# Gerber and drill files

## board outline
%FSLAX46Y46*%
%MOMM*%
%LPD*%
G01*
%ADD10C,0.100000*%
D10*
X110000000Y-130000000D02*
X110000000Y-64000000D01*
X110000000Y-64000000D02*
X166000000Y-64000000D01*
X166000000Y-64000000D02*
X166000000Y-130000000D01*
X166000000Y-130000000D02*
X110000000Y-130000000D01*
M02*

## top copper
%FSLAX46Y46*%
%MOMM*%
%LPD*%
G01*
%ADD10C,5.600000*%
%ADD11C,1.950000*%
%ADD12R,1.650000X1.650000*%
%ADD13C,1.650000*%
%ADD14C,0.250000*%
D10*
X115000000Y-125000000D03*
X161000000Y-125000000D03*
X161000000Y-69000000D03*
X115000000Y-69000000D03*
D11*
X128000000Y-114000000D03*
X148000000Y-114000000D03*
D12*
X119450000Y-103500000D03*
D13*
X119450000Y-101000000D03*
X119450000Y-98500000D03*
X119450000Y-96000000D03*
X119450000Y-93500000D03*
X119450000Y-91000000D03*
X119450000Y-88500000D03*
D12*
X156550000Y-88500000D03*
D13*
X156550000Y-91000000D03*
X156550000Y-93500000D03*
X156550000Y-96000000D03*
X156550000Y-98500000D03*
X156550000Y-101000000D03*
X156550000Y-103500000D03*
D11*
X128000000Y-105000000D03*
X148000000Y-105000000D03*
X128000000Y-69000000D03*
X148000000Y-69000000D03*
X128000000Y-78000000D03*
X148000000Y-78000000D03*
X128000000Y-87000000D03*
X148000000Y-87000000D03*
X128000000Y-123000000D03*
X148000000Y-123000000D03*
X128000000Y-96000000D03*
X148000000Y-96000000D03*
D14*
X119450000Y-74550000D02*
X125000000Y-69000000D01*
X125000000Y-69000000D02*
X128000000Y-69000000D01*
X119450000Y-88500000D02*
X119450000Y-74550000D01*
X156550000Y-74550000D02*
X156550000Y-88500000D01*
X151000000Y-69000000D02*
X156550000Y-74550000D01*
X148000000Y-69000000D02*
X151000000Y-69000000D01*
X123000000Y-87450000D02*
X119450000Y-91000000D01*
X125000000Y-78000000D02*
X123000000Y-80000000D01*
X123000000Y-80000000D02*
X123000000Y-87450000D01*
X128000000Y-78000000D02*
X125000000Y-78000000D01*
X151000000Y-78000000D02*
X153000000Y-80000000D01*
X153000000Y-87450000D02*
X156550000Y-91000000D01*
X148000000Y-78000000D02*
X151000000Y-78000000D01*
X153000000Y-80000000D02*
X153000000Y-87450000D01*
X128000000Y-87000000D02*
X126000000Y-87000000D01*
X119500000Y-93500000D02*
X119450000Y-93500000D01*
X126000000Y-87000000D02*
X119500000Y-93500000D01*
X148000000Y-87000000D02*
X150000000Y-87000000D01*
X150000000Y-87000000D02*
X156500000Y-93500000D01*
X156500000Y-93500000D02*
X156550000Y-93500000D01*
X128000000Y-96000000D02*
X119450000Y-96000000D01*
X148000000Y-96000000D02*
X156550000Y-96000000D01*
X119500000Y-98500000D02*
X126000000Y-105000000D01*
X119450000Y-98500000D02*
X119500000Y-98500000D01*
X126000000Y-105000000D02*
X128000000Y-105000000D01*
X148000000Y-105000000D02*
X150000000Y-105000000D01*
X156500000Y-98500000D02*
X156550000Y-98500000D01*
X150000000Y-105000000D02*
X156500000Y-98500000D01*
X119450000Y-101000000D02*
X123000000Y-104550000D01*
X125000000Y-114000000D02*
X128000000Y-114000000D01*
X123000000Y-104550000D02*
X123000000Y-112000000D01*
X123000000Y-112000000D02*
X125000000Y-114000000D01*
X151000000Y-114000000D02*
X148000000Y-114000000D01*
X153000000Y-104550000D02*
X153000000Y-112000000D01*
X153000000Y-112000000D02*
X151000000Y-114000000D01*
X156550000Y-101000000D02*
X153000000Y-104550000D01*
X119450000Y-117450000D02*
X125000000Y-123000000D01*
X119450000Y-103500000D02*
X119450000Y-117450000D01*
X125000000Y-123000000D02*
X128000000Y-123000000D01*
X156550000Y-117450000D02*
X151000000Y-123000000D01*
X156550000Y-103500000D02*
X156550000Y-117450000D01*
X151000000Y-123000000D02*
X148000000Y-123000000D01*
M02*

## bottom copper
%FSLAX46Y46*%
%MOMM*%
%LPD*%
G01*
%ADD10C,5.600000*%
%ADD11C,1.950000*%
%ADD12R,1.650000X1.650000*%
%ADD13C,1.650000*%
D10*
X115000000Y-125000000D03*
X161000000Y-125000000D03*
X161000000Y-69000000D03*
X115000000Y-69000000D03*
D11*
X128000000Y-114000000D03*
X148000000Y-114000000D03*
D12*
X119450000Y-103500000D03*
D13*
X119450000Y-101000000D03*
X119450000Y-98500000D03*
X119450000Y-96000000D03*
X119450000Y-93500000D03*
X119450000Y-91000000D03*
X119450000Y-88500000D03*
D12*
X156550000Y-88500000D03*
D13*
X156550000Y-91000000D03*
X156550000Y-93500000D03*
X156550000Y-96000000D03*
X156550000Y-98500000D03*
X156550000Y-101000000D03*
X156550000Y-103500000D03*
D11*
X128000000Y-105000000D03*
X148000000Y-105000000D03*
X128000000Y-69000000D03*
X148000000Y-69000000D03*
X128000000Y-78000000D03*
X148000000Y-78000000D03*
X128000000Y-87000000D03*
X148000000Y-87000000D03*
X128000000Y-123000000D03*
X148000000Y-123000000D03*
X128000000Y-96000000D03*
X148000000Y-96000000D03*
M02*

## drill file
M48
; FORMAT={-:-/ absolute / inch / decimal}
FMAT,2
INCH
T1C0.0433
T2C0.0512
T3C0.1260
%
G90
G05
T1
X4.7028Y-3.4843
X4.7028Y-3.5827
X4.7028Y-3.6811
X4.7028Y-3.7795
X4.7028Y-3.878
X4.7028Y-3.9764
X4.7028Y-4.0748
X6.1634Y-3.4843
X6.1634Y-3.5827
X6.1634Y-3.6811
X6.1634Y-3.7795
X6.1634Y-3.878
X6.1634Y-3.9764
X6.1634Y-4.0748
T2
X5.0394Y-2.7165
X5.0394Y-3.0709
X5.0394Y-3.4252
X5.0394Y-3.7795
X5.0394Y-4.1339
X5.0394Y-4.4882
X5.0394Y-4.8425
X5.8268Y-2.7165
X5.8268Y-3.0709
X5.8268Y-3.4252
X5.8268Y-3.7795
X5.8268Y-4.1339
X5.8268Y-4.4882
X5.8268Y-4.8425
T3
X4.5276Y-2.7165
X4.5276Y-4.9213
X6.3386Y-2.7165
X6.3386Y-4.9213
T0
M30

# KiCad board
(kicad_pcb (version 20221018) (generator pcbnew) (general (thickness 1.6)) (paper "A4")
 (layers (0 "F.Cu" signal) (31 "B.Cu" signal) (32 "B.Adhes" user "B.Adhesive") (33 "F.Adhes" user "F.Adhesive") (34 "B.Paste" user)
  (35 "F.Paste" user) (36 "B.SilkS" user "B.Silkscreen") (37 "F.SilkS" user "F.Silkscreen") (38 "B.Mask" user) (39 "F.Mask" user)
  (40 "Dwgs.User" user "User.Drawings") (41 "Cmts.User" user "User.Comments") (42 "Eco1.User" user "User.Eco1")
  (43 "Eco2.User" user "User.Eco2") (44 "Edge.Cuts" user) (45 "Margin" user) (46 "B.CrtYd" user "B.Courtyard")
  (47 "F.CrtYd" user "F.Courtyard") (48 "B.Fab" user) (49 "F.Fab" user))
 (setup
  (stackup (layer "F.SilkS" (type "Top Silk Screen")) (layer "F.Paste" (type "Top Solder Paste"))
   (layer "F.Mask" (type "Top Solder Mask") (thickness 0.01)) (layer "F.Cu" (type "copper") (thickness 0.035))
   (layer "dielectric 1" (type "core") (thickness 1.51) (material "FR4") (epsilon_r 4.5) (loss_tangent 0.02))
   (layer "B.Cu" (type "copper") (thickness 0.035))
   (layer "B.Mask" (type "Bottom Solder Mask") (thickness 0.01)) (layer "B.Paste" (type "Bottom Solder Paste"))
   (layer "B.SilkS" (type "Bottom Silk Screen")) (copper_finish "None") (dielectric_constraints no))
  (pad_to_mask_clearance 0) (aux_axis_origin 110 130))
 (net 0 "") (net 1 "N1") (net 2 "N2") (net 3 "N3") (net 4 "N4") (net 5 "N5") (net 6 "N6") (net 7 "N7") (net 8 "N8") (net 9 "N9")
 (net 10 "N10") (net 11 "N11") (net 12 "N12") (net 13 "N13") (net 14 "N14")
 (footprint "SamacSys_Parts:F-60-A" (layer "F.Cu") (at 138 114)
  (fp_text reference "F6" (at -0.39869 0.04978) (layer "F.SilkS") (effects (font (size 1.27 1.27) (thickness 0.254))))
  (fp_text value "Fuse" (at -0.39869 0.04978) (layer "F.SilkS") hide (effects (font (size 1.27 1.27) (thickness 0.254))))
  (pad "1" thru_hole circle (at -10 0) (size 1.95 1.95) (drill 1.3) (layers "*.Cu" "*.Mask") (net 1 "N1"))
  (pad "2" thru_hole circle (at 10 0) (size 1.95 1.95) (drill 1.3) (layers "*.Cu" "*.Mask") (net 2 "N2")))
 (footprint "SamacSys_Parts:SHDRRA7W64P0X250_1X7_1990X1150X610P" (layer "F.Cu") (at 119.45 103.5 90)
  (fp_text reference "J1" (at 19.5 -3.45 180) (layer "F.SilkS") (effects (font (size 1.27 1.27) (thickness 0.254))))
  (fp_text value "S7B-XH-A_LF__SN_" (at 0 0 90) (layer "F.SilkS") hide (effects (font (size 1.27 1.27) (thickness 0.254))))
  (pad "1" thru_hole rect (at 0 0 90) (size 1.65 1.65) (drill 1.1) (layers "*.Cu" "*.Mask") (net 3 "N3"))
  (pad "2" thru_hole circle (at 2.5 0 90) (size 1.65 1.65) (drill 1.1) (layers "*.Cu" "*.Mask") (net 1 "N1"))
  (pad "3" thru_hole circle (at 5 0 90) (size 1.65 1.65) (drill 1.1) (layers "*.Cu" "*.Mask") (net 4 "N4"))
  (pad "4" thru_hole circle (at 7.5 0 90) (size 1.65 1.65) (drill 1.1) (layers "*.Cu" "*.Mask") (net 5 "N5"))
  (pad "5" thru_hole circle (at 10 0 90) (size 1.65 1.65) (drill 1.1) (layers "*.Cu" "*.Mask") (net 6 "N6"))
  (pad "6" thru_hole circle (at 12.5 0 90) (size 1.65 1.65) (drill 1.1) (layers "*.Cu" "*.Mask") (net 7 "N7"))
  (pad "7" thru_hole circle (at 15 0 90) (size 1.65 1.65) (drill 1.1) (layers "*.Cu" "*.Mask") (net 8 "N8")))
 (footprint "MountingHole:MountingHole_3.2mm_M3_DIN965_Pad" (layer "F.Cu") (at 161 69)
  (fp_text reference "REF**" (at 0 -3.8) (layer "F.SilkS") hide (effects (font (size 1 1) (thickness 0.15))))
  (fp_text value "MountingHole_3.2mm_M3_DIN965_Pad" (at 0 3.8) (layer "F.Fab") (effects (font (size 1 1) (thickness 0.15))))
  (pad "1" thru_hole circle (at 0 0) (size 5.6 5.6) (drill 3.2) (layers "F&B.Cu" "*.Mask")))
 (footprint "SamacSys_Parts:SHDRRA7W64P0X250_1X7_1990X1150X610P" (layer "F.Cu") (at 156.55 88.5 -90)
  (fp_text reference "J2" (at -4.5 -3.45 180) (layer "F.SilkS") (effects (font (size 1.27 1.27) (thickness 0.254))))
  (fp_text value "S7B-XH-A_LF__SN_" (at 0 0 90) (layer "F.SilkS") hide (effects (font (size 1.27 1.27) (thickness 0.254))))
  (pad "1" thru_hole rect (at 0 0 270) (size 1.65 1.65) (drill 1.1) (layers "*.Cu" "*.Mask") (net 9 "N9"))
  (pad "2" thru_hole circle (at 2.5 0 270) (size 1.65 1.65) (drill 1.1) (layers "*.Cu" "*.Mask") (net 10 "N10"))
  (pad "3" thru_hole circle (at 5 0 270) (size 1.65 1.65) (drill 1.1) (layers "*.Cu" "*.Mask") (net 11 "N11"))
  (pad "4" thru_hole circle (at 7.5 0 270) (size 1.65 1.65) (drill 1.1) (layers "*.Cu" "*.Mask") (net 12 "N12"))
  (pad "5" thru_hole circle (at 10 0 270) (size 1.65 1.65) (drill 1.1) (layers "*.Cu" "*.Mask") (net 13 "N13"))
  (pad "6" thru_hole circle (at 12.5 0 270) (size 1.65 1.65) (drill 1.1) (layers "*.Cu" "*.Mask") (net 2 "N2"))
  (pad "7" thru_hole circle (at 15 0 270) (size 1.65 1.65) (drill 1.1) (layers "*.Cu" "*.Mask") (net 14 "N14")))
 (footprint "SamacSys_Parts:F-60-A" (layer "F.Cu") (at 138 105)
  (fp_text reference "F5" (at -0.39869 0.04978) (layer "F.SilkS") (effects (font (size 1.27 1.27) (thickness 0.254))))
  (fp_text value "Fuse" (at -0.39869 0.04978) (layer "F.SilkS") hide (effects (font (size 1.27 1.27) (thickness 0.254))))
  (pad "1" thru_hole circle (at -10 0) (size 1.95 1.95) (drill 1.3) (layers "*.Cu" "*.Mask") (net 4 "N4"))
  (pad "2" thru_hole circle (at 10 0) (size 1.95 1.95) (drill 1.3) (layers "*.Cu" "*.Mask") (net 13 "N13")))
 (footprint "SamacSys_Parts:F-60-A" (layer "F.Cu") (at 138 69)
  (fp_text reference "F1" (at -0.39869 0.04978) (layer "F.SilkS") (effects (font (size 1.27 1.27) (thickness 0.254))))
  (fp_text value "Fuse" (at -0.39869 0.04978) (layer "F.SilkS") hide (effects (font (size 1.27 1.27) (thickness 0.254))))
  (pad "1" thru_hole circle (at -10 0) (size 1.95 1.95) (drill 1.3) (layers "*.Cu" "*.Mask") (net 8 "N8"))
  (pad "2" thru_hole circle (at 10 0) (size 1.95 1.95) (drill 1.3) (layers "*.Cu" "*.Mask") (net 9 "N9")))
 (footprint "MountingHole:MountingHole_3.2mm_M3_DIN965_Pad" (layer "F.Cu") (at 115 125)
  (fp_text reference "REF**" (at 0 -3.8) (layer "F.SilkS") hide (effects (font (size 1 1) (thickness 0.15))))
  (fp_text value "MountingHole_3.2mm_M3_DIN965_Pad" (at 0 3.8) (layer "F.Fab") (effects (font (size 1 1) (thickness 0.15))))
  (pad "1" thru_hole circle (at 0 0) (size 5.6 5.6) (drill 3.2) (layers "F&B.Cu" "*.Mask")))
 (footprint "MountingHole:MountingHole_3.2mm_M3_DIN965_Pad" (layer "F.Cu") (at 115 69)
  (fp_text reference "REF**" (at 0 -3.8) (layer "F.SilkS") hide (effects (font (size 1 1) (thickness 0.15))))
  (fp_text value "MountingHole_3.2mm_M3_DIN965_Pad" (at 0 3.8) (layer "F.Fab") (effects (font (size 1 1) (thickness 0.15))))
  (pad "1" thru_hole circle (at 0 0) (size 5.6 5.6) (drill 3.2) (layers "*.Cu" "*.Mask")))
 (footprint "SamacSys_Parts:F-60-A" (layer "F.Cu") (at 138 78)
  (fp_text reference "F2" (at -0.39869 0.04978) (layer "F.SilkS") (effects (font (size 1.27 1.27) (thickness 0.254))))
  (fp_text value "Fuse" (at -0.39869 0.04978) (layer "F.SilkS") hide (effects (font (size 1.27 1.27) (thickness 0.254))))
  (pad "1" thru_hole circle (at -10 0) (size 1.95 1.95) (drill 1.3) (layers "*.Cu" "*.Mask") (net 7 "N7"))
  (pad "2" thru_hole circle (at 10 0) (size 1.95 1.95) (drill 1.3) (layers "*.Cu" "*.Mask") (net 10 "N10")))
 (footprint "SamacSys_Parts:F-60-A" (layer "F.Cu") (at 138 87)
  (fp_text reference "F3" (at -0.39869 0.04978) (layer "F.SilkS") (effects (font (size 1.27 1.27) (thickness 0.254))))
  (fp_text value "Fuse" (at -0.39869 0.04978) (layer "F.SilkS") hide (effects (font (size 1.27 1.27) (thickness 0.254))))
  (pad "1" thru_hole circle (at -10 0) (size 1.95 1.95) (drill 1.3) (layers "*.Cu" "*.Mask") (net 6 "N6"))
  (pad "2" thru_hole circle (at 10 0) (size 1.95 1.95) (drill 1.3) (layers "*.Cu" "*.Mask") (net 11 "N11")))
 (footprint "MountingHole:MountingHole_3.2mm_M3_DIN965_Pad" (layer "F.Cu") (at 161 125)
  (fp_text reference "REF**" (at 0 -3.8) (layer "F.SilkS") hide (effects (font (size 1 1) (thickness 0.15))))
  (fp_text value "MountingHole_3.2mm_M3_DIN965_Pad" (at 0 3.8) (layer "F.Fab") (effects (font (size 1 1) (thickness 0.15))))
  (pad "1" thru_hole circle (at 0 0) (size 5.6 5.6) (drill 3.2) (layers "F&B.Cu" "*.Mask")))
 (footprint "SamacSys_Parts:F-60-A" (layer "F.Cu") (at 138 123)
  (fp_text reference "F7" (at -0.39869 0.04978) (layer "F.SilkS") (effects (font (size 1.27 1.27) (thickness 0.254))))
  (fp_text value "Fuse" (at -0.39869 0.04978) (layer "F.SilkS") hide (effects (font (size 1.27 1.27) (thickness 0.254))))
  (pad "1" thru_hole circle (at -10 0) (size 1.95 1.95) (drill 1.3) (layers "*.Cu" "*.Mask") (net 3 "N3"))
  (pad "2" thru_hole circle (at 10 0) (size 1.95 1.95) (drill 1.3) (layers "*.Cu" "*.Mask") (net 14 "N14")))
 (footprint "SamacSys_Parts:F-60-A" (layer "F.Cu") (at 138 96)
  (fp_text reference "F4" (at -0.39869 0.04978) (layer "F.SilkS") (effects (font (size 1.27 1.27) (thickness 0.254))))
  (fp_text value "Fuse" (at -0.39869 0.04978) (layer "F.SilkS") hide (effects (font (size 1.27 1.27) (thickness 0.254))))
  (pad "1" thru_hole circle (at -10 0) (size 1.95 1.95) (drill 1.3) (layers "*.Cu" "*.Mask") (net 5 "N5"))
  (pad "2" thru_hole circle (at 10 0) (size 1.95 1.95) (drill 1.3) (layers "*.Cu" "*.Mask") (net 12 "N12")))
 (gr_line (start 110 130) (end 110 64) (stroke (width 0.1) (type solid)) (layer "Edge.Cuts"))
 (gr_line (start 110 64) (end 166 64) (stroke (width 0.1) (type solid)) (layer "Edge.Cuts"))
 (gr_line (start 166 64) (end 166 130) (stroke (width 0.1) (type solid)) (layer "Edge.Cuts"))
 (gr_line (start 166 130) (end 110 130) (stroke (width 0.1) (type solid)) (layer "Edge.Cuts"))
 (segment (start 119.45 74.55) (end 125 69) (width 0.25) (layer "F.Cu") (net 8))
 (segment (start 125 69) (end 128 69) (width 0.25) (layer "F.Cu") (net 8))
 (segment (start 119.45 88.5) (end 119.45 74.55) (width 0.25) (layer "F.Cu") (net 8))
 (segment (start 156.55 74.55) (end 156.55 88.5) (width 0.25) (layer "F.Cu") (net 9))
 (segment (start 151 69) (end 156.55 74.55) (width 0.25) (layer "F.Cu") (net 9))
 (segment (start 148 69) (end 151 69) (width 0.25) (layer "F.Cu") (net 9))
 (segment (start 123 87.45) (end 119.45 91) (width 0.25) (layer "F.Cu") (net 7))
 (segment (start 125 78) (end 123 80) (width 0.25) (layer "F.Cu") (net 7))
 (segment (start 123 80) (end 123 87.45) (width 0.25) (layer "F.Cu") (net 7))
 (segment (start 128 78) (end 125 78) (width 0.25) (layer "F.Cu") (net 7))
 (segment (start 151 78) (end 153 80) (width 0.25) (layer "F.Cu") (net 10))
 (segment (start 153 87.45) (end 156.55 91) (width 0.25) (layer "F.Cu") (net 10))
 (segment (start 148 78) (end 151 78) (width 0.25) (layer "F.Cu") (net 10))
 (segment (start 153 80) (end 153 87.45) (width 0.25) (layer "F.Cu") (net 10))
 (segment (start 128 87) (end 126 87) (width 0.25) (layer "F.Cu") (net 6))
 (segment (start 119.5 93.5) (end 119.45 93.5) (width 0.25) (layer "F.Cu") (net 6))
 (segment (start 126 87) (end 119.5 93.5) (width 0.25) (layer "F.Cu") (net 6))
 (segment (start 148 87) (end 150 87) (width 0.25) (layer "F.Cu") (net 11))
 (segment (start 150 87) (end 156.5 93.5) (width 0.25) (layer "F.Cu") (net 11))
 (segment (start 156.5 93.5) (end 156.55 93.5) (width 0.25) (layer "F.Cu") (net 11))
 (segment (start 128 96) (end 119.45 96) (width 0.25) (layer "F.Cu") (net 5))
 (segment (start 148 96) (end 156.55 96) (width 0.25) (layer "F.Cu") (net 12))
 (segment (start 119.5 98.5) (end 126 105) (width 0.25) (layer "F.Cu") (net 4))
 (segment (start 119.45 98.5) (end 119.5 98.5) (width 0.25) (layer "F.Cu") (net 4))
 (segment (start 126 105) (end 128 105) (width 0.25) (layer "F.Cu") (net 4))
 (segment (start 148 105) (end 150 105) (width 0.25) (layer "F.Cu") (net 13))
 (segment (start 156.5 98.5) (end 156.55 98.5) (width 0.25) (layer "F.Cu") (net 13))
 (segment (start 150 105) (end 156.5 98.5) (width 0.25) (layer "F.Cu") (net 13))
 (segment (start 119.45 101) (end 123 104.55) (width 0.25) (layer "F.Cu") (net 1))
 (segment (start 125 114) (end 128 114) (width 0.25) (layer "F.Cu") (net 1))
 (segment (start 123 104.55) (end 123 112) (width 0.25) (layer "F.Cu") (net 1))
 (segment (start 123 112) (end 125 114) (width 0.25) (layer "F.Cu") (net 1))
 (segment (start 151 114) (end 148 114) (width 0.25) (layer "F.Cu") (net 2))
 (segment (start 153 104.55) (end 153 112) (width 0.25) (layer "F.Cu") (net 2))
 (segment (start 153 112) (end 151 114) (width 0.25) (layer "F.Cu") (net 2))
 (segment (start 156.55 101) (end 153 104.55) (width 0.25) (layer "F.Cu") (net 2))
 (segment (start 119.45 117.45) (end 125 123) (width 0.25) (layer "F.Cu") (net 3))
 (segment (start 119.45 103.5) (end 119.45 117.45) (width 0.25) (layer "F.Cu") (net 3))
 (segment (start 125 123) (end 128 123) (width 0.25) (layer "F.Cu") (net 3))
 (segment (start 156.55 117.45) (end 151 123) (width 0.25) (layer "F.Cu") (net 14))
 (segment (start 156.55 103.5) (end 156.55 117.45) (width 0.25) (layer "F.Cu") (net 14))
 (segment (start 151 123) (end 148 123) (width 0.25) (layer "F.Cu") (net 14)))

